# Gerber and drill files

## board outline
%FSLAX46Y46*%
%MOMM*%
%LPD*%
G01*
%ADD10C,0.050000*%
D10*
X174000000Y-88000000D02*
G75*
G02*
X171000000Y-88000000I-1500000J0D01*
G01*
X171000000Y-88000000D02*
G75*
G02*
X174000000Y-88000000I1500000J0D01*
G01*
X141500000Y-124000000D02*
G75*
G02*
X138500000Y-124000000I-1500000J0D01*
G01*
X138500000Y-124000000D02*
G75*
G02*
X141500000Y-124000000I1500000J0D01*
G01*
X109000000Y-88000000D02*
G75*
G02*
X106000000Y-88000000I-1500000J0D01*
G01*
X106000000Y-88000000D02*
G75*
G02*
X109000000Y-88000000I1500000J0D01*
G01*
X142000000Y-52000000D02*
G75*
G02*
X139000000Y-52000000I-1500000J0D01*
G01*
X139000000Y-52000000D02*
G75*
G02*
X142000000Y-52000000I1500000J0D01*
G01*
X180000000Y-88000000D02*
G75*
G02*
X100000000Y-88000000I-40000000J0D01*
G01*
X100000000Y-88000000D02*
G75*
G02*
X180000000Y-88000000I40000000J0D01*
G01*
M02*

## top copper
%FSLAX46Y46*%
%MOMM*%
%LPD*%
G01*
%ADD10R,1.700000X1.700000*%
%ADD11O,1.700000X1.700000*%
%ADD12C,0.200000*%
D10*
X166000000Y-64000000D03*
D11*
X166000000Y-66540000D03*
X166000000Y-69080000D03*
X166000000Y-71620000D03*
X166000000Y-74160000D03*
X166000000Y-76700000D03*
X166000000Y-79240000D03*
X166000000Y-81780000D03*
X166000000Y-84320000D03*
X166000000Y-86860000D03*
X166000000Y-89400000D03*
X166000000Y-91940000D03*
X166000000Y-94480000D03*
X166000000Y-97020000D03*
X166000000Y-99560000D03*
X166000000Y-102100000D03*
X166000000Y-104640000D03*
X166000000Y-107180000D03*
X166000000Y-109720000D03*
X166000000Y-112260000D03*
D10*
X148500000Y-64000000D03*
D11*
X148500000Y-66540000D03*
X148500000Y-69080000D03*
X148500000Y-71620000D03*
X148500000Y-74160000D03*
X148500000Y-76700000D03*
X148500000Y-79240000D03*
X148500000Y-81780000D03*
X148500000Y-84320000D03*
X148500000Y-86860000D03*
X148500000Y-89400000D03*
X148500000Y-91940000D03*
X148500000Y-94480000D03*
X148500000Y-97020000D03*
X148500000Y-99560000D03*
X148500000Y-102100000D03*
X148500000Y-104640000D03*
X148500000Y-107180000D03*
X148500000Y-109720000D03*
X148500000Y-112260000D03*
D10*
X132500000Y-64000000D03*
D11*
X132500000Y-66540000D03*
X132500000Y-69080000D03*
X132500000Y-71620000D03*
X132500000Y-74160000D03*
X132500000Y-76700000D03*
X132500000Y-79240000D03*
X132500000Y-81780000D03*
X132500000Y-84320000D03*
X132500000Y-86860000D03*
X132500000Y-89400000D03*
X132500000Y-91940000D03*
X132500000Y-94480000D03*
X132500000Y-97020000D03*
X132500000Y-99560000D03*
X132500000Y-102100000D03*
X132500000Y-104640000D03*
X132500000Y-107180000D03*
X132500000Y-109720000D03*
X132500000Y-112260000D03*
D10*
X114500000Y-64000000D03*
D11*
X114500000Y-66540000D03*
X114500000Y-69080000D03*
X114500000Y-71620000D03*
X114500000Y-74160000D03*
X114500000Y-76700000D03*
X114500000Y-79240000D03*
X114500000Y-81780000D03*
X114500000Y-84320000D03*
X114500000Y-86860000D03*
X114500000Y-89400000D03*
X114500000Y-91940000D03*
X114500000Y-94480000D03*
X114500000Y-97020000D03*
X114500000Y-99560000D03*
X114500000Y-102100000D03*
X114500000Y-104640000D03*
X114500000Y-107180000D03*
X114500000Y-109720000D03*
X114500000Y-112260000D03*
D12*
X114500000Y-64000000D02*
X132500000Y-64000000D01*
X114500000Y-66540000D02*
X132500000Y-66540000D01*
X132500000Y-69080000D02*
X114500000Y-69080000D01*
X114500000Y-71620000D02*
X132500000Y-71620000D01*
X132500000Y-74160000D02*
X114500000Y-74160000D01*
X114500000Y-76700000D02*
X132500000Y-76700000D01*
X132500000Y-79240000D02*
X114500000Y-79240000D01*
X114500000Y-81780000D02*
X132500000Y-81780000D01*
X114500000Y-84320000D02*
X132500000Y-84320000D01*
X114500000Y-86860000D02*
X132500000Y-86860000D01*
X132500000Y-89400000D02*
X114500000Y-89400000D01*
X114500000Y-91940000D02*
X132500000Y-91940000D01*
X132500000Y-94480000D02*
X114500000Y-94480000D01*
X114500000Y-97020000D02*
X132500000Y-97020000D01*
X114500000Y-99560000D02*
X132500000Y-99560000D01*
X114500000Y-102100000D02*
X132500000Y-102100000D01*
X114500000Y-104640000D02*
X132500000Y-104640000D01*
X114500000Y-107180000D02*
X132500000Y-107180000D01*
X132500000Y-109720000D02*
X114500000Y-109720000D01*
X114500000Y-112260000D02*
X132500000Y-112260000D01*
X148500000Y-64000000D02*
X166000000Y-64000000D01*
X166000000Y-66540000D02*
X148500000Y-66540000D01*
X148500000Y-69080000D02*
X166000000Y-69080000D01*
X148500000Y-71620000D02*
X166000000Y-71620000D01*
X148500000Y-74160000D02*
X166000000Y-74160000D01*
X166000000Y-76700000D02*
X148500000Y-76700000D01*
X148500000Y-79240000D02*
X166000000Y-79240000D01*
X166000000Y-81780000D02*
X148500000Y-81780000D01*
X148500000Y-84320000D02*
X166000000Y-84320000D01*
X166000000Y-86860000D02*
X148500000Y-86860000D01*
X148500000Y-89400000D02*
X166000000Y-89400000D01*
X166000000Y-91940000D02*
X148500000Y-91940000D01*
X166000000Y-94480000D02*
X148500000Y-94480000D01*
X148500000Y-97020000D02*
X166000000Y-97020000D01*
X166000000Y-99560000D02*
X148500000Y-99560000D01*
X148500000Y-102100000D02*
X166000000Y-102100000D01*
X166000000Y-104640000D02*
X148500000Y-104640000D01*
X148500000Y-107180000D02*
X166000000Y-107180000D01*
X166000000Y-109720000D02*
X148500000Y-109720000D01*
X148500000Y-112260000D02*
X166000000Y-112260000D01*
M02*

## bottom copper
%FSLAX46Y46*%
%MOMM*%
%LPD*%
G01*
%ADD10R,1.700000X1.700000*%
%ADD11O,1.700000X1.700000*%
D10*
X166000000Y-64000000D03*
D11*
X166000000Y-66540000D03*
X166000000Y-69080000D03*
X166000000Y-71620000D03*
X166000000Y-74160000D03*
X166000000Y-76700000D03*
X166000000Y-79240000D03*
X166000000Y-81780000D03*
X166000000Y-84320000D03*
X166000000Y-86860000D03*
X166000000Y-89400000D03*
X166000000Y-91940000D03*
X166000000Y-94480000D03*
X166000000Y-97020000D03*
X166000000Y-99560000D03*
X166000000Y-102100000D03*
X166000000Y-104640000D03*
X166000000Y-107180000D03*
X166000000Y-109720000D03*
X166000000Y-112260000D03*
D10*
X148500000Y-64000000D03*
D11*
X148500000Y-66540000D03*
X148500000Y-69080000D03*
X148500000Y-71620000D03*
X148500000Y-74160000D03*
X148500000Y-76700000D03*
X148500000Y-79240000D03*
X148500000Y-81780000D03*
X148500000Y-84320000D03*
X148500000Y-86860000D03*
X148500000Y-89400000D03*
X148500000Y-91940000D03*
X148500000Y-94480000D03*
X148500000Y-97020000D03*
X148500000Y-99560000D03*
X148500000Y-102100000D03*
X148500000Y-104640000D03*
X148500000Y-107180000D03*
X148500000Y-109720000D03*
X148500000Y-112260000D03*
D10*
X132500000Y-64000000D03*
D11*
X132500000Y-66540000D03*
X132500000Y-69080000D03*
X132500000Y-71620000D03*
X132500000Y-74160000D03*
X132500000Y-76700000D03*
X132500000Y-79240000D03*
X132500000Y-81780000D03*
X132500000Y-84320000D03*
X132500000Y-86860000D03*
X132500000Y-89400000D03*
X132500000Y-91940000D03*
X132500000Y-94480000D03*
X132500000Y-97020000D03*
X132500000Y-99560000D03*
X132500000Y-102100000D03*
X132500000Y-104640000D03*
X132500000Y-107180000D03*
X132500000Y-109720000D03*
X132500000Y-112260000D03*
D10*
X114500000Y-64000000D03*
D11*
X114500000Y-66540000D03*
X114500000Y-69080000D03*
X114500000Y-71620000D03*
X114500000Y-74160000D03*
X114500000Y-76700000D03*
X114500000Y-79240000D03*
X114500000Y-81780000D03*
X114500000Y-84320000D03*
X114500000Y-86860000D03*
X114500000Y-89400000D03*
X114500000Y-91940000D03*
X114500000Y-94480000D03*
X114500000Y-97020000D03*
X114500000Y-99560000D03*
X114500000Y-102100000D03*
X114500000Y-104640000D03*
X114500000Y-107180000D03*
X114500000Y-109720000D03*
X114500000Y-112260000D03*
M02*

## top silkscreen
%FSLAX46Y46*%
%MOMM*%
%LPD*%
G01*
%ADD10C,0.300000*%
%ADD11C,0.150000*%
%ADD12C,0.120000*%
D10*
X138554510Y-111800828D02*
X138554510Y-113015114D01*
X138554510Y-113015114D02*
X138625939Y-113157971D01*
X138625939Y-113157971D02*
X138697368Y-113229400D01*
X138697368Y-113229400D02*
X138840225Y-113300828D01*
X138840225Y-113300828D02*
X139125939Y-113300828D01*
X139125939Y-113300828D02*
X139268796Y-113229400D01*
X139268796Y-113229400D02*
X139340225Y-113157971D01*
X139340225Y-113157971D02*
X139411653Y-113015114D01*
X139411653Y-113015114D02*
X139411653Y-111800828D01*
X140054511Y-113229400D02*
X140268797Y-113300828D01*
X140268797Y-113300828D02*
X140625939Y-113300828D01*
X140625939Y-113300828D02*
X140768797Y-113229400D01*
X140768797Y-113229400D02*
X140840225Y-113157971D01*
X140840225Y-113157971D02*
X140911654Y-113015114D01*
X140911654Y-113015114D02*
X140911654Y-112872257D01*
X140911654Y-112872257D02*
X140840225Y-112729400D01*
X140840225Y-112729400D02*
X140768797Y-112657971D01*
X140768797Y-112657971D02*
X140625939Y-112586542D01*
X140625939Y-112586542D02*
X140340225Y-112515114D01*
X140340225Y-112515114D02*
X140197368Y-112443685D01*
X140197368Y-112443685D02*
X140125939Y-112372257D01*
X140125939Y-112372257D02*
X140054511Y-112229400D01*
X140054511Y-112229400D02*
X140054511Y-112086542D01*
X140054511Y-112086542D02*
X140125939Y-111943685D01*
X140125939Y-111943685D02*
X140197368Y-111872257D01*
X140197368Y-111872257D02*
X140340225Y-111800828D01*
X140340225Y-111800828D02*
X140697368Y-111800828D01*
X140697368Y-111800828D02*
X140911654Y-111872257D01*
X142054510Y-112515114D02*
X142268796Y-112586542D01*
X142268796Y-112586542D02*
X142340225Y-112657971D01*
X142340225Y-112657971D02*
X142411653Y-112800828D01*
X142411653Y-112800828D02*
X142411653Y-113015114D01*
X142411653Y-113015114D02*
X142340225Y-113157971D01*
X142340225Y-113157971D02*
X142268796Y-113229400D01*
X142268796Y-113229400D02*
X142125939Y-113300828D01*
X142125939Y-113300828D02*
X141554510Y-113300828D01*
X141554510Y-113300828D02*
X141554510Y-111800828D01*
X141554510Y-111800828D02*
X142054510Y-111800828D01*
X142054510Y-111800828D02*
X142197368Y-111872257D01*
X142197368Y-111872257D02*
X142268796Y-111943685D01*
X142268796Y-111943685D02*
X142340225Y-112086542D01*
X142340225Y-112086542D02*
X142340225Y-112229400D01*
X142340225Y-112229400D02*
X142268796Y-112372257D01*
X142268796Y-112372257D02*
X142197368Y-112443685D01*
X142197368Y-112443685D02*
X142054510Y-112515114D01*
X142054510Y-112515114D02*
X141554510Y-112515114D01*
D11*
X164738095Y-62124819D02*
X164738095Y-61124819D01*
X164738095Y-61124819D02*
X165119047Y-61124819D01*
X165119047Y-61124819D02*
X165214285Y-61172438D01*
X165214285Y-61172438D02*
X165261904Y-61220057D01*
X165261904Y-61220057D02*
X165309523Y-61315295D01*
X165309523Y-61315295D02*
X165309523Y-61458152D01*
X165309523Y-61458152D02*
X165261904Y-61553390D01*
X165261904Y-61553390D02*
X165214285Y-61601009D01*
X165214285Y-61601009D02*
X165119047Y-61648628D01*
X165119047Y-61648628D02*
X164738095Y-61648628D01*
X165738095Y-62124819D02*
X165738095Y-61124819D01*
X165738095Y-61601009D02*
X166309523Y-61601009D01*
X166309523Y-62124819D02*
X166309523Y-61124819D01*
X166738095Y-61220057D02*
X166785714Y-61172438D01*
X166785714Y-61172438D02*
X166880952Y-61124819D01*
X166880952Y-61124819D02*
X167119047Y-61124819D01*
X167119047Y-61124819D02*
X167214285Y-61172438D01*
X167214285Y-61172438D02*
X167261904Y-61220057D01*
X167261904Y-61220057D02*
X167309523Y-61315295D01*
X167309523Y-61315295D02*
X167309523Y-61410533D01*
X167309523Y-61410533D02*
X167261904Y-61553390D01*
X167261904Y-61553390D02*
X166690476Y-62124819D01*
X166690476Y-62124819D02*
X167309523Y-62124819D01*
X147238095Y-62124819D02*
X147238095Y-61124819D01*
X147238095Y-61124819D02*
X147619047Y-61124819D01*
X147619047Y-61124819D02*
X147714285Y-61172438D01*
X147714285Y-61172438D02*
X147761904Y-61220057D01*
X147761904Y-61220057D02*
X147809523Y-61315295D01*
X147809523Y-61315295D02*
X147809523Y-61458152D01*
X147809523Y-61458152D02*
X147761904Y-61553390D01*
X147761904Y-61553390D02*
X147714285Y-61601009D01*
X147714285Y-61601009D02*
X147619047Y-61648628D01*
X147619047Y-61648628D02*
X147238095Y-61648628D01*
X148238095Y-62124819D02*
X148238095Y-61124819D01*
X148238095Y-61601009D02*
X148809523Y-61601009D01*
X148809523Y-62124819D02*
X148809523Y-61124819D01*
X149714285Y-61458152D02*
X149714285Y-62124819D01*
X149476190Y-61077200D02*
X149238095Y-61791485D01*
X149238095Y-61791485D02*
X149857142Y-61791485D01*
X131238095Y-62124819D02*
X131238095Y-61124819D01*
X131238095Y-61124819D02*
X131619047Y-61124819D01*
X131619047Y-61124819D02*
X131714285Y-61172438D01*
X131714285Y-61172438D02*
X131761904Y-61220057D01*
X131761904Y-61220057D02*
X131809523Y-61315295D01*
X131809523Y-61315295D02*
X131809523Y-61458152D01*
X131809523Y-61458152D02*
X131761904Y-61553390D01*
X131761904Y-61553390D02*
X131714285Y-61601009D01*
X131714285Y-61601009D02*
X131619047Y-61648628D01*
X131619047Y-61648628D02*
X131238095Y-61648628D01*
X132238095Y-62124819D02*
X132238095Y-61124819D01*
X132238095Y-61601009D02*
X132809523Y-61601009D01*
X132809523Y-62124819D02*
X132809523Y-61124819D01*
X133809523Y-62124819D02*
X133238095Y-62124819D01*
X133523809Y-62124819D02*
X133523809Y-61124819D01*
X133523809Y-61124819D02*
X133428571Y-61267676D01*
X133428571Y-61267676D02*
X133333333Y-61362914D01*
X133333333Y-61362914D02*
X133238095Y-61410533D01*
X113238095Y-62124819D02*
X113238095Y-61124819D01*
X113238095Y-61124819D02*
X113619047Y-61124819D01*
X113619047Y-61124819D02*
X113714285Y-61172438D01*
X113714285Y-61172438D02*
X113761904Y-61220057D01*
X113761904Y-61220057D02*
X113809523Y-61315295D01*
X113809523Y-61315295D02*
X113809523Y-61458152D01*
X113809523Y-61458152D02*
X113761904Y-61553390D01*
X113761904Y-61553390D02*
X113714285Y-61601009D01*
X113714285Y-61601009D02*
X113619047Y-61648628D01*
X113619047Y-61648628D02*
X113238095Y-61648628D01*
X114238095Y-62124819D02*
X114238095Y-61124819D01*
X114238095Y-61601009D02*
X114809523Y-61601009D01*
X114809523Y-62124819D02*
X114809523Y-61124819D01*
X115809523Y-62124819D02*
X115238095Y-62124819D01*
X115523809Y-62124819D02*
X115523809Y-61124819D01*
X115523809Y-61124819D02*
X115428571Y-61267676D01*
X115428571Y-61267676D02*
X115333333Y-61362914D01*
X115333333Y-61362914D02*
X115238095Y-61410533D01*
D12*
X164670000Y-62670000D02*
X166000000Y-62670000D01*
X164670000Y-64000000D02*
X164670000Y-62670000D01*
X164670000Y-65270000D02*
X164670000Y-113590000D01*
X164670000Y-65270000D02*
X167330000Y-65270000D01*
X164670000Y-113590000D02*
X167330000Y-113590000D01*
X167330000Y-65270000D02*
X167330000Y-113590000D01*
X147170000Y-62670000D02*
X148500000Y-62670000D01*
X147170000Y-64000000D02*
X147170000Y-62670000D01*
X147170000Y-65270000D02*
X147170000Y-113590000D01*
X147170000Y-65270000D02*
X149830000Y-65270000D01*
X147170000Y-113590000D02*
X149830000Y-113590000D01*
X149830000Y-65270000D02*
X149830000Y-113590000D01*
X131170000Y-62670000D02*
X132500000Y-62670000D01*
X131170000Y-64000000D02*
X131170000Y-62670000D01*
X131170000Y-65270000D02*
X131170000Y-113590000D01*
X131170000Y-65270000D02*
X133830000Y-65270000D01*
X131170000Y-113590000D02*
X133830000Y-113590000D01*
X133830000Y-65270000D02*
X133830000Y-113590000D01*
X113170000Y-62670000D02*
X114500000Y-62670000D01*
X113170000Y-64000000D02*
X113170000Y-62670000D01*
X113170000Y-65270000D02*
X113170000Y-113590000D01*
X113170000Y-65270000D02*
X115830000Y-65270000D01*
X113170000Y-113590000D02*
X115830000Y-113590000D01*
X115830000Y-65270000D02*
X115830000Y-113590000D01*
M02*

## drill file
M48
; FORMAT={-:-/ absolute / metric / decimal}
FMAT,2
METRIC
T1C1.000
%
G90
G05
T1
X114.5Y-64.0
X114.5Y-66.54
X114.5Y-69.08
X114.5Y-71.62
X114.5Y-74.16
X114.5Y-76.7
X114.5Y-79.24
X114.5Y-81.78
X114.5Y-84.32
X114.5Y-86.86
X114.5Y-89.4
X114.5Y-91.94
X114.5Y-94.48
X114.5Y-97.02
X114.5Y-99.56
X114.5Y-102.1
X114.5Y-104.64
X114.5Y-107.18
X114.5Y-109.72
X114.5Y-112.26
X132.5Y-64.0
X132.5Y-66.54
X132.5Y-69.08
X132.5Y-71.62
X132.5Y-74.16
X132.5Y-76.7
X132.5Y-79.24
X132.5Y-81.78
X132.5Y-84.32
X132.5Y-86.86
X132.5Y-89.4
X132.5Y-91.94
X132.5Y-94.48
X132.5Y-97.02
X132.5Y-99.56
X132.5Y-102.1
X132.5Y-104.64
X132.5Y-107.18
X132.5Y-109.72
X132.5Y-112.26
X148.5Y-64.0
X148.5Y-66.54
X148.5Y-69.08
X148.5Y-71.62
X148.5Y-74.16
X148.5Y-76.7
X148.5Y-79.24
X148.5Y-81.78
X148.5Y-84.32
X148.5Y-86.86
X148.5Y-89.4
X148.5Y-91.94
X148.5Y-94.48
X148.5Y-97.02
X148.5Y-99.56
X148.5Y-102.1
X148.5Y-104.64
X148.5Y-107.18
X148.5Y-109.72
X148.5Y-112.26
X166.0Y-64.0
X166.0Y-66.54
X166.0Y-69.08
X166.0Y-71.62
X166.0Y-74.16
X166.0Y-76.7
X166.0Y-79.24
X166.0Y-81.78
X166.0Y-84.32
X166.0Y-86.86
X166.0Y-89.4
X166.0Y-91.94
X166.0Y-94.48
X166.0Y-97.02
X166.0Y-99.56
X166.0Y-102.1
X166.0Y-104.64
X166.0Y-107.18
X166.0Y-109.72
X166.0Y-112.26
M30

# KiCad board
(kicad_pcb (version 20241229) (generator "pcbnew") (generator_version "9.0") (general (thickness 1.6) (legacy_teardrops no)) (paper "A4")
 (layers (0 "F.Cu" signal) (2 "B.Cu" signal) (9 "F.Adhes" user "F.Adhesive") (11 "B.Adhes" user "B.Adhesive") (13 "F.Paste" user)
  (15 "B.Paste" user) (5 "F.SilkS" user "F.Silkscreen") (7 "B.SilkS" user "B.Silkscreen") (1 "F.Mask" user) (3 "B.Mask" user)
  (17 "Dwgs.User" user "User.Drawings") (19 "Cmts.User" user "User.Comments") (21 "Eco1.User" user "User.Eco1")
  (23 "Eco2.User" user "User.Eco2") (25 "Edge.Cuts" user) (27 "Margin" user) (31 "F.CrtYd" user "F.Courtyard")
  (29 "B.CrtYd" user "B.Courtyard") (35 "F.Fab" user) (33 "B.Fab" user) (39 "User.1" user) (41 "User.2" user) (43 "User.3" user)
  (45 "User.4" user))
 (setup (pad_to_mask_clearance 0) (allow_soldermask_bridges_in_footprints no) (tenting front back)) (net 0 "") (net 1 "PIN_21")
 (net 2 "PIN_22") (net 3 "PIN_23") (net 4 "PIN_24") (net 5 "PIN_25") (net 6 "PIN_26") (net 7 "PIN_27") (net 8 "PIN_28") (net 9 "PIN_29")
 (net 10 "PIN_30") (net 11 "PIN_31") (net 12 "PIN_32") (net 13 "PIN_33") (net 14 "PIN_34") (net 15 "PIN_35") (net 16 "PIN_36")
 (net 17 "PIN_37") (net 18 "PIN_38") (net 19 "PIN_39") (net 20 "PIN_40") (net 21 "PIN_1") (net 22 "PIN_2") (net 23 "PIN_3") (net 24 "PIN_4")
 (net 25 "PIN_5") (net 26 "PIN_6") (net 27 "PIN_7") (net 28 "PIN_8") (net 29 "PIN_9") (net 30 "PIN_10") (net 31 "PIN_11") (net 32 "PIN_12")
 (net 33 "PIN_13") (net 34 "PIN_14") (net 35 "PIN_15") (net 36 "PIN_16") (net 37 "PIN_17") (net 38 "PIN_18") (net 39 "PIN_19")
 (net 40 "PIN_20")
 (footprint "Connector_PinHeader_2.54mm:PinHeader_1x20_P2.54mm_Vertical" (layer "F.Cu") (at 166 64)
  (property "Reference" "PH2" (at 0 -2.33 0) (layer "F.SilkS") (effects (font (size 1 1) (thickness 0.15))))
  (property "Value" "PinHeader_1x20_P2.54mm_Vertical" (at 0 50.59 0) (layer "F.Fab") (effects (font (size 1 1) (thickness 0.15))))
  (fp_line (start -1.33 -1.33) (end 0 -1.33) (stroke (width 0.12) (type solid)) (layer "F.SilkS"))
  (fp_line (start -1.33 0) (end -1.33 -1.33) (stroke (width 0.12) (type solid)) (layer "F.SilkS"))
  (fp_line (start -1.33 1.27) (end -1.33 49.59) (stroke (width 0.12) (type solid)) (layer "F.SilkS"))
  (fp_line (start -1.33 1.27) (end 1.33 1.27) (stroke (width 0.12) (type solid)) (layer "F.SilkS"))
  (fp_line (start -1.33 49.59) (end 1.33 49.59) (stroke (width 0.12) (type solid)) (layer "F.SilkS"))
  (fp_line (start 1.33 1.27) (end 1.33 49.59) (stroke (width 0.12) (type solid)) (layer "F.SilkS"))
  (pad "1" thru_hole rect (at 0 0) (size 1.7 1.7) (drill 1) (layers "*.Cu" "*.Mask") (remove_unused_layers no) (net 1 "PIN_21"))
  (pad "2" thru_hole oval (at 0 2.54) (size 1.7 1.7) (drill 1) (layers "*.Cu" "*.Mask") (remove_unused_layers no) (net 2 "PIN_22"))
  (pad "3" thru_hole oval (at 0 5.08) (size 1.7 1.7) (drill 1) (layers "*.Cu" "*.Mask") (remove_unused_layers no) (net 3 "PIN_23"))
  (pad "4" thru_hole oval (at 0 7.62) (size 1.7 1.7) (drill 1) (layers "*.Cu" "*.Mask") (remove_unused_layers no) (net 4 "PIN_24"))
  (pad "5" thru_hole oval (at 0 10.16) (size 1.7 1.7) (drill 1) (layers "*.Cu" "*.Mask") (remove_unused_layers no) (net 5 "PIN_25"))
  (pad "6" thru_hole oval (at 0 12.7) (size 1.7 1.7) (drill 1) (layers "*.Cu" "*.Mask") (remove_unused_layers no) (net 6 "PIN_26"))
  (pad "7" thru_hole oval (at 0 15.24) (size 1.7 1.7) (drill 1) (layers "*.Cu" "*.Mask") (remove_unused_layers no) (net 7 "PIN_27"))
  (pad "8" thru_hole oval (at 0 17.78) (size 1.7 1.7) (drill 1) (layers "*.Cu" "*.Mask") (remove_unused_layers no) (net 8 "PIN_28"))
  (pad "9" thru_hole oval (at 0 20.32) (size 1.7 1.7) (drill 1) (layers "*.Cu" "*.Mask") (remove_unused_layers no) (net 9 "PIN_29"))
  (pad "10" thru_hole oval (at 0 22.86) (size 1.7 1.7) (drill 1) (layers "*.Cu" "*.Mask") (remove_unused_layers no) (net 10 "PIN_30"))
  (pad "11" thru_hole oval (at 0 25.4) (size 1.7 1.7) (drill 1) (layers "*.Cu" "*.Mask") (remove_unused_layers no) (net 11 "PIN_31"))
  (pad "12" thru_hole oval (at 0 27.94) (size 1.7 1.7) (drill 1) (layers "*.Cu" "*.Mask") (remove_unused_layers no) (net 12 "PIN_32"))
  (pad "13" thru_hole oval (at 0 30.48) (size 1.7 1.7) (drill 1) (layers "*.Cu" "*.Mask") (remove_unused_layers no) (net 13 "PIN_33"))
  (pad "14" thru_hole oval (at 0 33.02) (size 1.7 1.7) (drill 1) (layers "*.Cu" "*.Mask") (remove_unused_layers no) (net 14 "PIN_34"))
  (pad "15" thru_hole oval (at 0 35.56) (size 1.7 1.7) (drill 1) (layers "*.Cu" "*.Mask") (remove_unused_layers no) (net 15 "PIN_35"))
  (pad "16" thru_hole oval (at 0 38.1) (size 1.7 1.7) (drill 1) (layers "*.Cu" "*.Mask") (remove_unused_layers no) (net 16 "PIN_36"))
  (pad "17" thru_hole oval (at 0 40.64) (size 1.7 1.7) (drill 1) (layers "*.Cu" "*.Mask") (remove_unused_layers no) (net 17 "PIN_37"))
  (pad "18" thru_hole oval (at 0 43.18) (size 1.7 1.7) (drill 1) (layers "*.Cu" "*.Mask") (remove_unused_layers no) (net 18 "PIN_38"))
  (pad "19" thru_hole oval (at 0 45.72) (size 1.7 1.7) (drill 1) (layers "*.Cu" "*.Mask") (remove_unused_layers no) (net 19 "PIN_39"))
  (pad "20" thru_hole oval (at 0 48.26) (size 1.7 1.7) (drill 1) (layers "*.Cu" "*.Mask") (remove_unused_layers no) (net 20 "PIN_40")))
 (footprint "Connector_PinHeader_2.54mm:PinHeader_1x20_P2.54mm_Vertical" (layer "F.Cu") (at 148.5 64)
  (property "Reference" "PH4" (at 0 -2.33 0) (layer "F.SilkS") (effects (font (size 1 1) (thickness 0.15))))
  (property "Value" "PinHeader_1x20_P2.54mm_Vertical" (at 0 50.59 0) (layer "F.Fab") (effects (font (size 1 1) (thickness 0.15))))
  (fp_line (start -1.33 -1.33) (end 0 -1.33) (stroke (width 0.12) (type solid)) (layer "F.SilkS"))
  (fp_line (start -1.33 0) (end -1.33 -1.33) (stroke (width 0.12) (type solid)) (layer "F.SilkS"))
  (fp_line (start -1.33 1.27) (end -1.33 49.59) (stroke (width 0.12) (type solid)) (layer "F.SilkS"))
  (fp_line (start -1.33 1.27) (end 1.33 1.27) (stroke (width 0.12) (type solid)) (layer "F.SilkS"))
  (fp_line (start -1.33 49.59) (end 1.33 49.59) (stroke (width 0.12) (type solid)) (layer "F.SilkS"))
  (fp_line (start 1.33 1.27) (end 1.33 49.59) (stroke (width 0.12) (type solid)) (layer "F.SilkS"))
  (pad "1" thru_hole rect (at 0 0) (size 1.7 1.7) (drill 1) (layers "*.Cu" "*.Mask") (remove_unused_layers no) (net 1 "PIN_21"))
  (pad "2" thru_hole oval (at 0 2.54) (size 1.7 1.7) (drill 1) (layers "*.Cu" "*.Mask") (remove_unused_layers no) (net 2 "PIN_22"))
  (pad "3" thru_hole oval (at 0 5.08) (size 1.7 1.7) (drill 1) (layers "*.Cu" "*.Mask") (remove_unused_layers no) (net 3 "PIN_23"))
  (pad "4" thru_hole oval (at 0 7.62) (size 1.7 1.7) (drill 1) (layers "*.Cu" "*.Mask") (remove_unused_layers no) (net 4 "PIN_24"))
  (pad "5" thru_hole oval (at 0 10.16) (size 1.7 1.7) (drill 1) (layers "*.Cu" "*.Mask") (remove_unused_layers no) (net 5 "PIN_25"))
  (pad "6" thru_hole oval (at 0 12.7) (size 1.7 1.7) (drill 1) (layers "*.Cu" "*.Mask") (remove_unused_layers no) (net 6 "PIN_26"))
  (pad "7" thru_hole oval (at 0 15.24) (size 1.7 1.7) (drill 1) (layers "*.Cu" "*.Mask") (remove_unused_layers no) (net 7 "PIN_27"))
  (pad "8" thru_hole oval (at 0 17.78) (size 1.7 1.7) (drill 1) (layers "*.Cu" "*.Mask") (remove_unused_layers no) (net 8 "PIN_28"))
  (pad "9" thru_hole oval (at 0 20.32) (size 1.7 1.7) (drill 1) (layers "*.Cu" "*.Mask") (remove_unused_layers no) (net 9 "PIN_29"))
  (pad "10" thru_hole oval (at 0 22.86) (size 1.7 1.7) (drill 1) (layers "*.Cu" "*.Mask") (remove_unused_layers no) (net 10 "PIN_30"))
  (pad "11" thru_hole oval (at 0 25.4) (size 1.7 1.7) (drill 1) (layers "*.Cu" "*.Mask") (remove_unused_layers no) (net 11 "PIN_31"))
  (pad "12" thru_hole oval (at 0 27.94) (size 1.7 1.7) (drill 1) (layers "*.Cu" "*.Mask") (remove_unused_layers no) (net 12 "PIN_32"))
  (pad "13" thru_hole oval (at 0 30.48) (size 1.7 1.7) (drill 1) (layers "*.Cu" "*.Mask") (remove_unused_layers no) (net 13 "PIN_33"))
  (pad "14" thru_hole oval (at 0 33.02) (size 1.7 1.7) (drill 1) (layers "*.Cu" "*.Mask") (remove_unused_layers no) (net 14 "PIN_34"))
  (pad "15" thru_hole oval (at 0 35.56) (size 1.7 1.7) (drill 1) (layers "*.Cu" "*.Mask") (remove_unused_layers no) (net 15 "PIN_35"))
  (pad "16" thru_hole oval (at 0 38.1) (size 1.7 1.7) (drill 1) (layers "*.Cu" "*.Mask") (remove_unused_layers no) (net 16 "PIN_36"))
  (pad "17" thru_hole oval (at 0 40.64) (size 1.7 1.7) (drill 1) (layers "*.Cu" "*.Mask") (remove_unused_layers no) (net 17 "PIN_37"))
  (pad "18" thru_hole oval (at 0 43.18) (size 1.7 1.7) (drill 1) (layers "*.Cu" "*.Mask") (remove_unused_layers no) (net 18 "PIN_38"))
  (pad "19" thru_hole oval (at 0 45.72) (size 1.7 1.7) (drill 1) (layers "*.Cu" "*.Mask") (remove_unused_layers no) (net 19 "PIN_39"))
  (pad "20" thru_hole oval (at 0 48.26) (size 1.7 1.7) (drill 1) (layers "*.Cu" "*.Mask") (remove_unused_layers no) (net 20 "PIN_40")))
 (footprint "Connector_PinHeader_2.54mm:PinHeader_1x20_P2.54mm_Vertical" (layer "F.Cu") (at 132.5 64)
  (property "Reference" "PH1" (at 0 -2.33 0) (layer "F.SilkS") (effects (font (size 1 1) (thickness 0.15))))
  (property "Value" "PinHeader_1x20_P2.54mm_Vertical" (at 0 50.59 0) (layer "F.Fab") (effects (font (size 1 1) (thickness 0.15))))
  (fp_line (start -1.33 -1.33) (end 0 -1.33) (stroke (width 0.12) (type solid)) (layer "F.SilkS"))
  (fp_line (start -1.33 0) (end -1.33 -1.33) (stroke (width 0.12) (type solid)) (layer "F.SilkS"))
  (fp_line (start -1.33 1.27) (end -1.33 49.59) (stroke (width 0.12) (type solid)) (layer "F.SilkS"))
  (fp_line (start -1.33 1.27) (end 1.33 1.27) (stroke (width 0.12) (type solid)) (layer "F.SilkS"))
  (fp_line (start -1.33 49.59) (end 1.33 49.59) (stroke (width 0.12) (type solid)) (layer "F.SilkS"))
  (fp_line (start 1.33 1.27) (end 1.33 49.59) (stroke (width 0.12) (type solid)) (layer "F.SilkS"))
  (pad "1" thru_hole rect (at 0 0) (size 1.7 1.7) (drill 1) (layers "*.Cu" "*.Mask") (remove_unused_layers no) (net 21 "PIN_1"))
  (pad "2" thru_hole oval (at 0 2.54) (size 1.7 1.7) (drill 1) (layers "*.Cu" "*.Mask") (remove_unused_layers no) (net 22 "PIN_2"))
  (pad "3" thru_hole oval (at 0 5.08) (size 1.7 1.7) (drill 1) (layers "*.Cu" "*.Mask") (remove_unused_layers no) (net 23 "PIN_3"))
  (pad "4" thru_hole oval (at 0 7.62) (size 1.7 1.7) (drill 1) (layers "*.Cu" "*.Mask") (remove_unused_layers no) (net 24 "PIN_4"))
  (pad "5" thru_hole oval (at 0 10.16) (size 1.7 1.7) (drill 1) (layers "*.Cu" "*.Mask") (remove_unused_layers no) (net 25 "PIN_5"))
  (pad "6" thru_hole oval (at 0 12.7) (size 1.7 1.7) (drill 1) (layers "*.Cu" "*.Mask") (remove_unused_layers no) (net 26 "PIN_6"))
  (pad "7" thru_hole oval (at 0 15.24) (size 1.7 1.7) (drill 1) (layers "*.Cu" "*.Mask") (remove_unused_layers no) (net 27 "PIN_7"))
  (pad "8" thru_hole oval (at 0 17.78) (size 1.7 1.7) (drill 1) (layers "*.Cu" "*.Mask") (remove_unused_layers no) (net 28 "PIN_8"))
  (pad "9" thru_hole oval (at 0 20.32) (size 1.7 1.7) (drill 1) (layers "*.Cu" "*.Mask") (remove_unused_layers no) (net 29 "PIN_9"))
  (pad "10" thru_hole oval (at 0 22.86) (size 1.7 1.7) (drill 1) (layers "*.Cu" "*.Mask") (remove_unused_layers no) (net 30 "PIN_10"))
  (pad "11" thru_hole oval (at 0 25.4) (size 1.7 1.7) (drill 1) (layers "*.Cu" "*.Mask") (remove_unused_layers no) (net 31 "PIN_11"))
  (pad "12" thru_hole oval (at 0 27.94) (size 1.7 1.7) (drill 1) (layers "*.Cu" "*.Mask") (remove_unused_layers no) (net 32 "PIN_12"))
  (pad "13" thru_hole oval (at 0 30.48) (size 1.7 1.7) (drill 1) (layers "*.Cu" "*.Mask") (remove_unused_layers no) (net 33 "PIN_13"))
  (pad "14" thru_hole oval (at 0 33.02) (size 1.7 1.7) (drill 1) (layers "*.Cu" "*.Mask") (remove_unused_layers no) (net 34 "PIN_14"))
  (pad "15" thru_hole oval (at 0 35.56) (size 1.7 1.7) (drill 1) (layers "*.Cu" "*.Mask") (remove_unused_layers no) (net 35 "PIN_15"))
  (pad "16" thru_hole oval (at 0 38.1) (size 1.7 1.7) (drill 1) (layers "*.Cu" "*.Mask") (remove_unused_layers no) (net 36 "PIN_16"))
  (pad "17" thru_hole oval (at 0 40.64) (size 1.7 1.7) (drill 1) (layers "*.Cu" "*.Mask") (remove_unused_layers no) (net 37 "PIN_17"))
  (pad "18" thru_hole oval (at 0 43.18) (size 1.7 1.7) (drill 1) (layers "*.Cu" "*.Mask") (remove_unused_layers no) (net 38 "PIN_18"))
  (pad "19" thru_hole oval (at 0 45.72) (size 1.7 1.7) (drill 1) (layers "*.Cu" "*.Mask") (remove_unused_layers no) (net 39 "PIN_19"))
  (pad "20" thru_hole oval (at 0 48.26) (size 1.7 1.7) (drill 1) (layers "*.Cu" "*.Mask") (remove_unused_layers no) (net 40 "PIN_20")))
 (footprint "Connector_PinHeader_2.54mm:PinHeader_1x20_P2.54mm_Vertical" (layer "F.Cu") (at 114.5 64)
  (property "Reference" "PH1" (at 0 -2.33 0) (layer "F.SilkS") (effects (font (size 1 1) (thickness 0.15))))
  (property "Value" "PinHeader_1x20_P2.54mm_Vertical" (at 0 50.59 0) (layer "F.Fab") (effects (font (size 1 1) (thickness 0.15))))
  (fp_line (start -1.33 -1.33) (end 0 -1.33) (stroke (width 0.12) (type solid)) (layer "F.SilkS"))
  (fp_line (start -1.33 0) (end -1.33 -1.33) (stroke (width 0.12) (type solid)) (layer "F.SilkS"))
  (fp_line (start -1.33 1.27) (end -1.33 49.59) (stroke (width 0.12) (type solid)) (layer "F.SilkS"))
  (fp_line (start -1.33 1.27) (end 1.33 1.27) (stroke (width 0.12) (type solid)) (layer "F.SilkS"))
  (fp_line (start -1.33 49.59) (end 1.33 49.59) (stroke (width 0.12) (type solid)) (layer "F.SilkS"))
  (fp_line (start 1.33 1.27) (end 1.33 49.59) (stroke (width 0.12) (type solid)) (layer "F.SilkS"))
  (pad "1" thru_hole rect (at 0 0) (size 1.7 1.7) (drill 1) (layers "*.Cu" "*.Mask") (remove_unused_layers no) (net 21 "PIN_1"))
  (pad "2" thru_hole oval (at 0 2.54) (size 1.7 1.7) (drill 1) (layers "*.Cu" "*.Mask") (remove_unused_layers no) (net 22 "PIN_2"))
  (pad "3" thru_hole oval (at 0 5.08) (size 1.7 1.7) (drill 1) (layers "*.Cu" "*.Mask") (remove_unused_layers no) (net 23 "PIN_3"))
  (pad "4" thru_hole oval (at 0 7.62) (size 1.7 1.7) (drill 1) (layers "*.Cu" "*.Mask") (remove_unused_layers no) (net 24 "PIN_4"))
  (pad "5" thru_hole oval (at 0 10.16) (size 1.7 1.7) (drill 1) (layers "*.Cu" "*.Mask") (remove_unused_layers no) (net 25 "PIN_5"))
  (pad "6" thru_hole oval (at 0 12.7) (size 1.7 1.7) (drill 1) (layers "*.Cu" "*.Mask") (remove_unused_layers no) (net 26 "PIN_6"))
  (pad "7" thru_hole oval (at 0 15.24) (size 1.7 1.7) (drill 1) (layers "*.Cu" "*.Mask") (remove_unused_layers no) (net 27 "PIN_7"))
  (pad "8" thru_hole oval (at 0 17.78) (size 1.7 1.7) (drill 1) (layers "*.Cu" "*.Mask") (remove_unused_layers no) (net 28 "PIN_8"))
  (pad "9" thru_hole oval (at 0 20.32) (size 1.7 1.7) (drill 1) (layers "*.Cu" "*.Mask") (remove_unused_layers no) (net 29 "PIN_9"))
  (pad "10" thru_hole oval (at 0 22.86) (size 1.7 1.7) (drill 1) (layers "*.Cu" "*.Mask") (remove_unused_layers no) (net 30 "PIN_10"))
  (pad "11" thru_hole oval (at 0 25.4) (size 1.7 1.7) (drill 1) (layers "*.Cu" "*.Mask") (remove_unused_layers no) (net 31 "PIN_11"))
  (pad "12" thru_hole oval (at 0 27.94) (size 1.7 1.7) (drill 1) (layers "*.Cu" "*.Mask") (remove_unused_layers no) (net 32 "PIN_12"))
  (pad "13" thru_hole oval (at 0 30.48) (size 1.7 1.7) (drill 1) (layers "*.Cu" "*.Mask") (remove_unused_layers no) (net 33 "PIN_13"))
  (pad "14" thru_hole oval (at 0 33.02) (size 1.7 1.7) (drill 1) (layers "*.Cu" "*.Mask") (remove_unused_layers no) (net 34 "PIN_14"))
  (pad "15" thru_hole oval (at 0 35.56) (size 1.7 1.7) (drill 1) (layers "*.Cu" "*.Mask") (remove_unused_layers no) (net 35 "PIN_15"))
  (pad "16" thru_hole oval (at 0 38.1) (size 1.7 1.7) (drill 1) (layers "*.Cu" "*.Mask") (remove_unused_layers no) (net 36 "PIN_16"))
  (pad "17" thru_hole oval (at 0 40.64) (size 1.7 1.7) (drill 1) (layers "*.Cu" "*.Mask") (remove_unused_layers no) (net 37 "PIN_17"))
  (pad "18" thru_hole oval (at 0 43.18) (size 1.7 1.7) (drill 1) (layers "*.Cu" "*.Mask") (remove_unused_layers no) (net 38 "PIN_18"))
  (pad "19" thru_hole oval (at 0 45.72) (size 1.7 1.7) (drill 1) (layers "*.Cu" "*.Mask") (remove_unused_layers no) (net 39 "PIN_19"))
  (pad "20" thru_hole oval (at 0 48.26) (size 1.7 1.7) (drill 1) (layers "*.Cu" "*.Mask") (remove_unused_layers no) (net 40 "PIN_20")))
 (gr_circle (center 172.5 88) (end 174 88) (stroke (width 0.05) (type default)) (fill no) (layer "Edge.Cuts"))
 (gr_circle (center 140 124) (end 141.5 124) (stroke (width 0.05) (type default)) (fill no) (layer "Edge.Cuts"))
 (gr_circle (center 107.5 88) (end 109 88) (stroke (width 0.05) (type default)) (fill no) (layer "Edge.Cuts"))
 (gr_circle (center 140.5 52) (end 142 52) (stroke (width 0.05) (type default)) (fill no) (layer "Edge.Cuts"))
 (gr_circle (center 140 88) (end 180 88) (stroke (width 0.05) (type default)) (fill no) (layer "Edge.Cuts"))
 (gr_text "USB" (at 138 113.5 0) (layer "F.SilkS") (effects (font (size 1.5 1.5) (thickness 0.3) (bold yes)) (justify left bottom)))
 (segment (start 114.5 64) (end 132.5 64) (width 0.2) (layer "F.Cu") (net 21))
 (segment (start 114.5 66.54) (end 132.5 66.54) (width 0.2) (layer "F.Cu") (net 22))
 (segment (start 132.5 69.08) (end 114.5 69.08) (width 0.2) (layer "F.Cu") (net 23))
 (segment (start 114.5 71.62) (end 132.5 71.62) (width 0.2) (layer "F.Cu") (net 24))
 (segment (start 132.5 74.16) (end 114.5 74.16) (width 0.2) (layer "F.Cu") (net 25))
 (segment (start 114.5 76.7) (end 132.5 76.7) (width 0.2) (layer "F.Cu") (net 26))
 (segment (start 132.5 79.24) (end 114.5 79.24) (width 0.2) (layer "F.Cu") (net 27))
 (segment (start 114.5 81.78) (end 132.5 81.78) (width 0.2) (layer "F.Cu") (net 28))
 (segment (start 114.5 84.32) (end 132.5 84.32) (width 0.2) (layer "F.Cu") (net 29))
 (segment (start 114.5 86.86) (end 132.5 86.86) (width 0.2) (layer "F.Cu") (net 30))
 (segment (start 132.5 89.4) (end 114.5 89.4) (width 0.2) (layer "F.Cu") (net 31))
 (segment (start 114.5 91.94) (end 132.5 91.94) (width 0.2) (layer "F.Cu") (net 32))
 (segment (start 132.5 94.48) (end 114.5 94.48) (width 0.2) (layer "F.Cu") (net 33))
 (segment (start 114.5 97.02) (end 132.5 97.02) (width 0.2) (layer "F.Cu") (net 34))
 (segment (start 114.5 99.56) (end 132.5 99.56) (width 0.2) (layer "F.Cu") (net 35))
 (segment (start 114.5 102.1) (end 132.5 102.1) (width 0.2) (layer "F.Cu") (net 36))
 (segment (start 114.5 104.64) (end 132.5 104.64) (width 0.2) (layer "F.Cu") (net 37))
 (segment (start 114.5 107.18) (end 132.5 107.18) (width 0.2) (layer "F.Cu") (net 38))
 (segment (start 132.5 109.72) (end 114.5 109.72) (width 0.2) (layer "F.Cu") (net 39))
 (segment (start 114.5 112.26) (end 132.5 112.26) (width 0.2) (layer "F.Cu") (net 40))
 (segment (start 148.5 64) (end 166 64) (width 0.2) (layer "F.Cu") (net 1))
 (segment (start 166 66.54) (end 148.5 66.54) (width 0.2) (layer "F.Cu") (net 2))
 (segment (start 148.5 69.08) (end 166 69.08) (width 0.2) (layer "F.Cu") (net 3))
 (segment (start 148.5 71.62) (end 166 71.62) (width 0.2) (layer "F.Cu") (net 4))
 (segment (start 148.5 74.16) (end 166 74.16) (width 0.2) (layer "F.Cu") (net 5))
 (segment (start 166 76.7) (end 148.5 76.7) (width 0.2) (layer "F.Cu") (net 6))
 (segment (start 148.5 79.24) (end 166 79.24) (width 0.2) (layer "F.Cu") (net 7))
 (segment (start 166 81.78) (end 148.5 81.78) (width 0.2) (layer "F.Cu") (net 8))
 (segment (start 148.5 84.32) (end 166 84.32) (width 0.2) (layer "F.Cu") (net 9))
 (segment (start 166 86.86) (end 148.5 86.86) (width 0.2) (layer "F.Cu") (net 10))
 (segment (start 148.5 89.4) (end 166 89.4) (width 0.2) (layer "F.Cu") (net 11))
 (segment (start 166 91.94) (end 148.5 91.94) (width 0.2) (layer "F.Cu") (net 12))
 (segment (start 166 94.48) (end 148.5 94.48) (width 0.2) (layer "F.Cu") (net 13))
 (segment (start 148.5 97.02) (end 166 97.02) (width 0.2) (layer "F.Cu") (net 14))
 (segment (start 166 99.56) (end 148.5 99.56) (width 0.2) (layer "F.Cu") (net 15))
 (segment (start 148.5 102.1) (end 166 102.1) (width 0.2) (layer "F.Cu") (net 16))
 (segment (start 166 104.64) (end 148.5 104.64) (width 0.2) (layer "F.Cu") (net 17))
 (segment (start 148.5 107.18) (end 166 107.18) (width 0.2) (layer "F.Cu") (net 18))
 (segment (start 166 109.72) (end 148.5 109.72) (width 0.2) (layer "F.Cu") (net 19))
 (segment (start 148.5 112.26) (end 166 112.26) (width 0.2) (layer "F.Cu") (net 20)))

